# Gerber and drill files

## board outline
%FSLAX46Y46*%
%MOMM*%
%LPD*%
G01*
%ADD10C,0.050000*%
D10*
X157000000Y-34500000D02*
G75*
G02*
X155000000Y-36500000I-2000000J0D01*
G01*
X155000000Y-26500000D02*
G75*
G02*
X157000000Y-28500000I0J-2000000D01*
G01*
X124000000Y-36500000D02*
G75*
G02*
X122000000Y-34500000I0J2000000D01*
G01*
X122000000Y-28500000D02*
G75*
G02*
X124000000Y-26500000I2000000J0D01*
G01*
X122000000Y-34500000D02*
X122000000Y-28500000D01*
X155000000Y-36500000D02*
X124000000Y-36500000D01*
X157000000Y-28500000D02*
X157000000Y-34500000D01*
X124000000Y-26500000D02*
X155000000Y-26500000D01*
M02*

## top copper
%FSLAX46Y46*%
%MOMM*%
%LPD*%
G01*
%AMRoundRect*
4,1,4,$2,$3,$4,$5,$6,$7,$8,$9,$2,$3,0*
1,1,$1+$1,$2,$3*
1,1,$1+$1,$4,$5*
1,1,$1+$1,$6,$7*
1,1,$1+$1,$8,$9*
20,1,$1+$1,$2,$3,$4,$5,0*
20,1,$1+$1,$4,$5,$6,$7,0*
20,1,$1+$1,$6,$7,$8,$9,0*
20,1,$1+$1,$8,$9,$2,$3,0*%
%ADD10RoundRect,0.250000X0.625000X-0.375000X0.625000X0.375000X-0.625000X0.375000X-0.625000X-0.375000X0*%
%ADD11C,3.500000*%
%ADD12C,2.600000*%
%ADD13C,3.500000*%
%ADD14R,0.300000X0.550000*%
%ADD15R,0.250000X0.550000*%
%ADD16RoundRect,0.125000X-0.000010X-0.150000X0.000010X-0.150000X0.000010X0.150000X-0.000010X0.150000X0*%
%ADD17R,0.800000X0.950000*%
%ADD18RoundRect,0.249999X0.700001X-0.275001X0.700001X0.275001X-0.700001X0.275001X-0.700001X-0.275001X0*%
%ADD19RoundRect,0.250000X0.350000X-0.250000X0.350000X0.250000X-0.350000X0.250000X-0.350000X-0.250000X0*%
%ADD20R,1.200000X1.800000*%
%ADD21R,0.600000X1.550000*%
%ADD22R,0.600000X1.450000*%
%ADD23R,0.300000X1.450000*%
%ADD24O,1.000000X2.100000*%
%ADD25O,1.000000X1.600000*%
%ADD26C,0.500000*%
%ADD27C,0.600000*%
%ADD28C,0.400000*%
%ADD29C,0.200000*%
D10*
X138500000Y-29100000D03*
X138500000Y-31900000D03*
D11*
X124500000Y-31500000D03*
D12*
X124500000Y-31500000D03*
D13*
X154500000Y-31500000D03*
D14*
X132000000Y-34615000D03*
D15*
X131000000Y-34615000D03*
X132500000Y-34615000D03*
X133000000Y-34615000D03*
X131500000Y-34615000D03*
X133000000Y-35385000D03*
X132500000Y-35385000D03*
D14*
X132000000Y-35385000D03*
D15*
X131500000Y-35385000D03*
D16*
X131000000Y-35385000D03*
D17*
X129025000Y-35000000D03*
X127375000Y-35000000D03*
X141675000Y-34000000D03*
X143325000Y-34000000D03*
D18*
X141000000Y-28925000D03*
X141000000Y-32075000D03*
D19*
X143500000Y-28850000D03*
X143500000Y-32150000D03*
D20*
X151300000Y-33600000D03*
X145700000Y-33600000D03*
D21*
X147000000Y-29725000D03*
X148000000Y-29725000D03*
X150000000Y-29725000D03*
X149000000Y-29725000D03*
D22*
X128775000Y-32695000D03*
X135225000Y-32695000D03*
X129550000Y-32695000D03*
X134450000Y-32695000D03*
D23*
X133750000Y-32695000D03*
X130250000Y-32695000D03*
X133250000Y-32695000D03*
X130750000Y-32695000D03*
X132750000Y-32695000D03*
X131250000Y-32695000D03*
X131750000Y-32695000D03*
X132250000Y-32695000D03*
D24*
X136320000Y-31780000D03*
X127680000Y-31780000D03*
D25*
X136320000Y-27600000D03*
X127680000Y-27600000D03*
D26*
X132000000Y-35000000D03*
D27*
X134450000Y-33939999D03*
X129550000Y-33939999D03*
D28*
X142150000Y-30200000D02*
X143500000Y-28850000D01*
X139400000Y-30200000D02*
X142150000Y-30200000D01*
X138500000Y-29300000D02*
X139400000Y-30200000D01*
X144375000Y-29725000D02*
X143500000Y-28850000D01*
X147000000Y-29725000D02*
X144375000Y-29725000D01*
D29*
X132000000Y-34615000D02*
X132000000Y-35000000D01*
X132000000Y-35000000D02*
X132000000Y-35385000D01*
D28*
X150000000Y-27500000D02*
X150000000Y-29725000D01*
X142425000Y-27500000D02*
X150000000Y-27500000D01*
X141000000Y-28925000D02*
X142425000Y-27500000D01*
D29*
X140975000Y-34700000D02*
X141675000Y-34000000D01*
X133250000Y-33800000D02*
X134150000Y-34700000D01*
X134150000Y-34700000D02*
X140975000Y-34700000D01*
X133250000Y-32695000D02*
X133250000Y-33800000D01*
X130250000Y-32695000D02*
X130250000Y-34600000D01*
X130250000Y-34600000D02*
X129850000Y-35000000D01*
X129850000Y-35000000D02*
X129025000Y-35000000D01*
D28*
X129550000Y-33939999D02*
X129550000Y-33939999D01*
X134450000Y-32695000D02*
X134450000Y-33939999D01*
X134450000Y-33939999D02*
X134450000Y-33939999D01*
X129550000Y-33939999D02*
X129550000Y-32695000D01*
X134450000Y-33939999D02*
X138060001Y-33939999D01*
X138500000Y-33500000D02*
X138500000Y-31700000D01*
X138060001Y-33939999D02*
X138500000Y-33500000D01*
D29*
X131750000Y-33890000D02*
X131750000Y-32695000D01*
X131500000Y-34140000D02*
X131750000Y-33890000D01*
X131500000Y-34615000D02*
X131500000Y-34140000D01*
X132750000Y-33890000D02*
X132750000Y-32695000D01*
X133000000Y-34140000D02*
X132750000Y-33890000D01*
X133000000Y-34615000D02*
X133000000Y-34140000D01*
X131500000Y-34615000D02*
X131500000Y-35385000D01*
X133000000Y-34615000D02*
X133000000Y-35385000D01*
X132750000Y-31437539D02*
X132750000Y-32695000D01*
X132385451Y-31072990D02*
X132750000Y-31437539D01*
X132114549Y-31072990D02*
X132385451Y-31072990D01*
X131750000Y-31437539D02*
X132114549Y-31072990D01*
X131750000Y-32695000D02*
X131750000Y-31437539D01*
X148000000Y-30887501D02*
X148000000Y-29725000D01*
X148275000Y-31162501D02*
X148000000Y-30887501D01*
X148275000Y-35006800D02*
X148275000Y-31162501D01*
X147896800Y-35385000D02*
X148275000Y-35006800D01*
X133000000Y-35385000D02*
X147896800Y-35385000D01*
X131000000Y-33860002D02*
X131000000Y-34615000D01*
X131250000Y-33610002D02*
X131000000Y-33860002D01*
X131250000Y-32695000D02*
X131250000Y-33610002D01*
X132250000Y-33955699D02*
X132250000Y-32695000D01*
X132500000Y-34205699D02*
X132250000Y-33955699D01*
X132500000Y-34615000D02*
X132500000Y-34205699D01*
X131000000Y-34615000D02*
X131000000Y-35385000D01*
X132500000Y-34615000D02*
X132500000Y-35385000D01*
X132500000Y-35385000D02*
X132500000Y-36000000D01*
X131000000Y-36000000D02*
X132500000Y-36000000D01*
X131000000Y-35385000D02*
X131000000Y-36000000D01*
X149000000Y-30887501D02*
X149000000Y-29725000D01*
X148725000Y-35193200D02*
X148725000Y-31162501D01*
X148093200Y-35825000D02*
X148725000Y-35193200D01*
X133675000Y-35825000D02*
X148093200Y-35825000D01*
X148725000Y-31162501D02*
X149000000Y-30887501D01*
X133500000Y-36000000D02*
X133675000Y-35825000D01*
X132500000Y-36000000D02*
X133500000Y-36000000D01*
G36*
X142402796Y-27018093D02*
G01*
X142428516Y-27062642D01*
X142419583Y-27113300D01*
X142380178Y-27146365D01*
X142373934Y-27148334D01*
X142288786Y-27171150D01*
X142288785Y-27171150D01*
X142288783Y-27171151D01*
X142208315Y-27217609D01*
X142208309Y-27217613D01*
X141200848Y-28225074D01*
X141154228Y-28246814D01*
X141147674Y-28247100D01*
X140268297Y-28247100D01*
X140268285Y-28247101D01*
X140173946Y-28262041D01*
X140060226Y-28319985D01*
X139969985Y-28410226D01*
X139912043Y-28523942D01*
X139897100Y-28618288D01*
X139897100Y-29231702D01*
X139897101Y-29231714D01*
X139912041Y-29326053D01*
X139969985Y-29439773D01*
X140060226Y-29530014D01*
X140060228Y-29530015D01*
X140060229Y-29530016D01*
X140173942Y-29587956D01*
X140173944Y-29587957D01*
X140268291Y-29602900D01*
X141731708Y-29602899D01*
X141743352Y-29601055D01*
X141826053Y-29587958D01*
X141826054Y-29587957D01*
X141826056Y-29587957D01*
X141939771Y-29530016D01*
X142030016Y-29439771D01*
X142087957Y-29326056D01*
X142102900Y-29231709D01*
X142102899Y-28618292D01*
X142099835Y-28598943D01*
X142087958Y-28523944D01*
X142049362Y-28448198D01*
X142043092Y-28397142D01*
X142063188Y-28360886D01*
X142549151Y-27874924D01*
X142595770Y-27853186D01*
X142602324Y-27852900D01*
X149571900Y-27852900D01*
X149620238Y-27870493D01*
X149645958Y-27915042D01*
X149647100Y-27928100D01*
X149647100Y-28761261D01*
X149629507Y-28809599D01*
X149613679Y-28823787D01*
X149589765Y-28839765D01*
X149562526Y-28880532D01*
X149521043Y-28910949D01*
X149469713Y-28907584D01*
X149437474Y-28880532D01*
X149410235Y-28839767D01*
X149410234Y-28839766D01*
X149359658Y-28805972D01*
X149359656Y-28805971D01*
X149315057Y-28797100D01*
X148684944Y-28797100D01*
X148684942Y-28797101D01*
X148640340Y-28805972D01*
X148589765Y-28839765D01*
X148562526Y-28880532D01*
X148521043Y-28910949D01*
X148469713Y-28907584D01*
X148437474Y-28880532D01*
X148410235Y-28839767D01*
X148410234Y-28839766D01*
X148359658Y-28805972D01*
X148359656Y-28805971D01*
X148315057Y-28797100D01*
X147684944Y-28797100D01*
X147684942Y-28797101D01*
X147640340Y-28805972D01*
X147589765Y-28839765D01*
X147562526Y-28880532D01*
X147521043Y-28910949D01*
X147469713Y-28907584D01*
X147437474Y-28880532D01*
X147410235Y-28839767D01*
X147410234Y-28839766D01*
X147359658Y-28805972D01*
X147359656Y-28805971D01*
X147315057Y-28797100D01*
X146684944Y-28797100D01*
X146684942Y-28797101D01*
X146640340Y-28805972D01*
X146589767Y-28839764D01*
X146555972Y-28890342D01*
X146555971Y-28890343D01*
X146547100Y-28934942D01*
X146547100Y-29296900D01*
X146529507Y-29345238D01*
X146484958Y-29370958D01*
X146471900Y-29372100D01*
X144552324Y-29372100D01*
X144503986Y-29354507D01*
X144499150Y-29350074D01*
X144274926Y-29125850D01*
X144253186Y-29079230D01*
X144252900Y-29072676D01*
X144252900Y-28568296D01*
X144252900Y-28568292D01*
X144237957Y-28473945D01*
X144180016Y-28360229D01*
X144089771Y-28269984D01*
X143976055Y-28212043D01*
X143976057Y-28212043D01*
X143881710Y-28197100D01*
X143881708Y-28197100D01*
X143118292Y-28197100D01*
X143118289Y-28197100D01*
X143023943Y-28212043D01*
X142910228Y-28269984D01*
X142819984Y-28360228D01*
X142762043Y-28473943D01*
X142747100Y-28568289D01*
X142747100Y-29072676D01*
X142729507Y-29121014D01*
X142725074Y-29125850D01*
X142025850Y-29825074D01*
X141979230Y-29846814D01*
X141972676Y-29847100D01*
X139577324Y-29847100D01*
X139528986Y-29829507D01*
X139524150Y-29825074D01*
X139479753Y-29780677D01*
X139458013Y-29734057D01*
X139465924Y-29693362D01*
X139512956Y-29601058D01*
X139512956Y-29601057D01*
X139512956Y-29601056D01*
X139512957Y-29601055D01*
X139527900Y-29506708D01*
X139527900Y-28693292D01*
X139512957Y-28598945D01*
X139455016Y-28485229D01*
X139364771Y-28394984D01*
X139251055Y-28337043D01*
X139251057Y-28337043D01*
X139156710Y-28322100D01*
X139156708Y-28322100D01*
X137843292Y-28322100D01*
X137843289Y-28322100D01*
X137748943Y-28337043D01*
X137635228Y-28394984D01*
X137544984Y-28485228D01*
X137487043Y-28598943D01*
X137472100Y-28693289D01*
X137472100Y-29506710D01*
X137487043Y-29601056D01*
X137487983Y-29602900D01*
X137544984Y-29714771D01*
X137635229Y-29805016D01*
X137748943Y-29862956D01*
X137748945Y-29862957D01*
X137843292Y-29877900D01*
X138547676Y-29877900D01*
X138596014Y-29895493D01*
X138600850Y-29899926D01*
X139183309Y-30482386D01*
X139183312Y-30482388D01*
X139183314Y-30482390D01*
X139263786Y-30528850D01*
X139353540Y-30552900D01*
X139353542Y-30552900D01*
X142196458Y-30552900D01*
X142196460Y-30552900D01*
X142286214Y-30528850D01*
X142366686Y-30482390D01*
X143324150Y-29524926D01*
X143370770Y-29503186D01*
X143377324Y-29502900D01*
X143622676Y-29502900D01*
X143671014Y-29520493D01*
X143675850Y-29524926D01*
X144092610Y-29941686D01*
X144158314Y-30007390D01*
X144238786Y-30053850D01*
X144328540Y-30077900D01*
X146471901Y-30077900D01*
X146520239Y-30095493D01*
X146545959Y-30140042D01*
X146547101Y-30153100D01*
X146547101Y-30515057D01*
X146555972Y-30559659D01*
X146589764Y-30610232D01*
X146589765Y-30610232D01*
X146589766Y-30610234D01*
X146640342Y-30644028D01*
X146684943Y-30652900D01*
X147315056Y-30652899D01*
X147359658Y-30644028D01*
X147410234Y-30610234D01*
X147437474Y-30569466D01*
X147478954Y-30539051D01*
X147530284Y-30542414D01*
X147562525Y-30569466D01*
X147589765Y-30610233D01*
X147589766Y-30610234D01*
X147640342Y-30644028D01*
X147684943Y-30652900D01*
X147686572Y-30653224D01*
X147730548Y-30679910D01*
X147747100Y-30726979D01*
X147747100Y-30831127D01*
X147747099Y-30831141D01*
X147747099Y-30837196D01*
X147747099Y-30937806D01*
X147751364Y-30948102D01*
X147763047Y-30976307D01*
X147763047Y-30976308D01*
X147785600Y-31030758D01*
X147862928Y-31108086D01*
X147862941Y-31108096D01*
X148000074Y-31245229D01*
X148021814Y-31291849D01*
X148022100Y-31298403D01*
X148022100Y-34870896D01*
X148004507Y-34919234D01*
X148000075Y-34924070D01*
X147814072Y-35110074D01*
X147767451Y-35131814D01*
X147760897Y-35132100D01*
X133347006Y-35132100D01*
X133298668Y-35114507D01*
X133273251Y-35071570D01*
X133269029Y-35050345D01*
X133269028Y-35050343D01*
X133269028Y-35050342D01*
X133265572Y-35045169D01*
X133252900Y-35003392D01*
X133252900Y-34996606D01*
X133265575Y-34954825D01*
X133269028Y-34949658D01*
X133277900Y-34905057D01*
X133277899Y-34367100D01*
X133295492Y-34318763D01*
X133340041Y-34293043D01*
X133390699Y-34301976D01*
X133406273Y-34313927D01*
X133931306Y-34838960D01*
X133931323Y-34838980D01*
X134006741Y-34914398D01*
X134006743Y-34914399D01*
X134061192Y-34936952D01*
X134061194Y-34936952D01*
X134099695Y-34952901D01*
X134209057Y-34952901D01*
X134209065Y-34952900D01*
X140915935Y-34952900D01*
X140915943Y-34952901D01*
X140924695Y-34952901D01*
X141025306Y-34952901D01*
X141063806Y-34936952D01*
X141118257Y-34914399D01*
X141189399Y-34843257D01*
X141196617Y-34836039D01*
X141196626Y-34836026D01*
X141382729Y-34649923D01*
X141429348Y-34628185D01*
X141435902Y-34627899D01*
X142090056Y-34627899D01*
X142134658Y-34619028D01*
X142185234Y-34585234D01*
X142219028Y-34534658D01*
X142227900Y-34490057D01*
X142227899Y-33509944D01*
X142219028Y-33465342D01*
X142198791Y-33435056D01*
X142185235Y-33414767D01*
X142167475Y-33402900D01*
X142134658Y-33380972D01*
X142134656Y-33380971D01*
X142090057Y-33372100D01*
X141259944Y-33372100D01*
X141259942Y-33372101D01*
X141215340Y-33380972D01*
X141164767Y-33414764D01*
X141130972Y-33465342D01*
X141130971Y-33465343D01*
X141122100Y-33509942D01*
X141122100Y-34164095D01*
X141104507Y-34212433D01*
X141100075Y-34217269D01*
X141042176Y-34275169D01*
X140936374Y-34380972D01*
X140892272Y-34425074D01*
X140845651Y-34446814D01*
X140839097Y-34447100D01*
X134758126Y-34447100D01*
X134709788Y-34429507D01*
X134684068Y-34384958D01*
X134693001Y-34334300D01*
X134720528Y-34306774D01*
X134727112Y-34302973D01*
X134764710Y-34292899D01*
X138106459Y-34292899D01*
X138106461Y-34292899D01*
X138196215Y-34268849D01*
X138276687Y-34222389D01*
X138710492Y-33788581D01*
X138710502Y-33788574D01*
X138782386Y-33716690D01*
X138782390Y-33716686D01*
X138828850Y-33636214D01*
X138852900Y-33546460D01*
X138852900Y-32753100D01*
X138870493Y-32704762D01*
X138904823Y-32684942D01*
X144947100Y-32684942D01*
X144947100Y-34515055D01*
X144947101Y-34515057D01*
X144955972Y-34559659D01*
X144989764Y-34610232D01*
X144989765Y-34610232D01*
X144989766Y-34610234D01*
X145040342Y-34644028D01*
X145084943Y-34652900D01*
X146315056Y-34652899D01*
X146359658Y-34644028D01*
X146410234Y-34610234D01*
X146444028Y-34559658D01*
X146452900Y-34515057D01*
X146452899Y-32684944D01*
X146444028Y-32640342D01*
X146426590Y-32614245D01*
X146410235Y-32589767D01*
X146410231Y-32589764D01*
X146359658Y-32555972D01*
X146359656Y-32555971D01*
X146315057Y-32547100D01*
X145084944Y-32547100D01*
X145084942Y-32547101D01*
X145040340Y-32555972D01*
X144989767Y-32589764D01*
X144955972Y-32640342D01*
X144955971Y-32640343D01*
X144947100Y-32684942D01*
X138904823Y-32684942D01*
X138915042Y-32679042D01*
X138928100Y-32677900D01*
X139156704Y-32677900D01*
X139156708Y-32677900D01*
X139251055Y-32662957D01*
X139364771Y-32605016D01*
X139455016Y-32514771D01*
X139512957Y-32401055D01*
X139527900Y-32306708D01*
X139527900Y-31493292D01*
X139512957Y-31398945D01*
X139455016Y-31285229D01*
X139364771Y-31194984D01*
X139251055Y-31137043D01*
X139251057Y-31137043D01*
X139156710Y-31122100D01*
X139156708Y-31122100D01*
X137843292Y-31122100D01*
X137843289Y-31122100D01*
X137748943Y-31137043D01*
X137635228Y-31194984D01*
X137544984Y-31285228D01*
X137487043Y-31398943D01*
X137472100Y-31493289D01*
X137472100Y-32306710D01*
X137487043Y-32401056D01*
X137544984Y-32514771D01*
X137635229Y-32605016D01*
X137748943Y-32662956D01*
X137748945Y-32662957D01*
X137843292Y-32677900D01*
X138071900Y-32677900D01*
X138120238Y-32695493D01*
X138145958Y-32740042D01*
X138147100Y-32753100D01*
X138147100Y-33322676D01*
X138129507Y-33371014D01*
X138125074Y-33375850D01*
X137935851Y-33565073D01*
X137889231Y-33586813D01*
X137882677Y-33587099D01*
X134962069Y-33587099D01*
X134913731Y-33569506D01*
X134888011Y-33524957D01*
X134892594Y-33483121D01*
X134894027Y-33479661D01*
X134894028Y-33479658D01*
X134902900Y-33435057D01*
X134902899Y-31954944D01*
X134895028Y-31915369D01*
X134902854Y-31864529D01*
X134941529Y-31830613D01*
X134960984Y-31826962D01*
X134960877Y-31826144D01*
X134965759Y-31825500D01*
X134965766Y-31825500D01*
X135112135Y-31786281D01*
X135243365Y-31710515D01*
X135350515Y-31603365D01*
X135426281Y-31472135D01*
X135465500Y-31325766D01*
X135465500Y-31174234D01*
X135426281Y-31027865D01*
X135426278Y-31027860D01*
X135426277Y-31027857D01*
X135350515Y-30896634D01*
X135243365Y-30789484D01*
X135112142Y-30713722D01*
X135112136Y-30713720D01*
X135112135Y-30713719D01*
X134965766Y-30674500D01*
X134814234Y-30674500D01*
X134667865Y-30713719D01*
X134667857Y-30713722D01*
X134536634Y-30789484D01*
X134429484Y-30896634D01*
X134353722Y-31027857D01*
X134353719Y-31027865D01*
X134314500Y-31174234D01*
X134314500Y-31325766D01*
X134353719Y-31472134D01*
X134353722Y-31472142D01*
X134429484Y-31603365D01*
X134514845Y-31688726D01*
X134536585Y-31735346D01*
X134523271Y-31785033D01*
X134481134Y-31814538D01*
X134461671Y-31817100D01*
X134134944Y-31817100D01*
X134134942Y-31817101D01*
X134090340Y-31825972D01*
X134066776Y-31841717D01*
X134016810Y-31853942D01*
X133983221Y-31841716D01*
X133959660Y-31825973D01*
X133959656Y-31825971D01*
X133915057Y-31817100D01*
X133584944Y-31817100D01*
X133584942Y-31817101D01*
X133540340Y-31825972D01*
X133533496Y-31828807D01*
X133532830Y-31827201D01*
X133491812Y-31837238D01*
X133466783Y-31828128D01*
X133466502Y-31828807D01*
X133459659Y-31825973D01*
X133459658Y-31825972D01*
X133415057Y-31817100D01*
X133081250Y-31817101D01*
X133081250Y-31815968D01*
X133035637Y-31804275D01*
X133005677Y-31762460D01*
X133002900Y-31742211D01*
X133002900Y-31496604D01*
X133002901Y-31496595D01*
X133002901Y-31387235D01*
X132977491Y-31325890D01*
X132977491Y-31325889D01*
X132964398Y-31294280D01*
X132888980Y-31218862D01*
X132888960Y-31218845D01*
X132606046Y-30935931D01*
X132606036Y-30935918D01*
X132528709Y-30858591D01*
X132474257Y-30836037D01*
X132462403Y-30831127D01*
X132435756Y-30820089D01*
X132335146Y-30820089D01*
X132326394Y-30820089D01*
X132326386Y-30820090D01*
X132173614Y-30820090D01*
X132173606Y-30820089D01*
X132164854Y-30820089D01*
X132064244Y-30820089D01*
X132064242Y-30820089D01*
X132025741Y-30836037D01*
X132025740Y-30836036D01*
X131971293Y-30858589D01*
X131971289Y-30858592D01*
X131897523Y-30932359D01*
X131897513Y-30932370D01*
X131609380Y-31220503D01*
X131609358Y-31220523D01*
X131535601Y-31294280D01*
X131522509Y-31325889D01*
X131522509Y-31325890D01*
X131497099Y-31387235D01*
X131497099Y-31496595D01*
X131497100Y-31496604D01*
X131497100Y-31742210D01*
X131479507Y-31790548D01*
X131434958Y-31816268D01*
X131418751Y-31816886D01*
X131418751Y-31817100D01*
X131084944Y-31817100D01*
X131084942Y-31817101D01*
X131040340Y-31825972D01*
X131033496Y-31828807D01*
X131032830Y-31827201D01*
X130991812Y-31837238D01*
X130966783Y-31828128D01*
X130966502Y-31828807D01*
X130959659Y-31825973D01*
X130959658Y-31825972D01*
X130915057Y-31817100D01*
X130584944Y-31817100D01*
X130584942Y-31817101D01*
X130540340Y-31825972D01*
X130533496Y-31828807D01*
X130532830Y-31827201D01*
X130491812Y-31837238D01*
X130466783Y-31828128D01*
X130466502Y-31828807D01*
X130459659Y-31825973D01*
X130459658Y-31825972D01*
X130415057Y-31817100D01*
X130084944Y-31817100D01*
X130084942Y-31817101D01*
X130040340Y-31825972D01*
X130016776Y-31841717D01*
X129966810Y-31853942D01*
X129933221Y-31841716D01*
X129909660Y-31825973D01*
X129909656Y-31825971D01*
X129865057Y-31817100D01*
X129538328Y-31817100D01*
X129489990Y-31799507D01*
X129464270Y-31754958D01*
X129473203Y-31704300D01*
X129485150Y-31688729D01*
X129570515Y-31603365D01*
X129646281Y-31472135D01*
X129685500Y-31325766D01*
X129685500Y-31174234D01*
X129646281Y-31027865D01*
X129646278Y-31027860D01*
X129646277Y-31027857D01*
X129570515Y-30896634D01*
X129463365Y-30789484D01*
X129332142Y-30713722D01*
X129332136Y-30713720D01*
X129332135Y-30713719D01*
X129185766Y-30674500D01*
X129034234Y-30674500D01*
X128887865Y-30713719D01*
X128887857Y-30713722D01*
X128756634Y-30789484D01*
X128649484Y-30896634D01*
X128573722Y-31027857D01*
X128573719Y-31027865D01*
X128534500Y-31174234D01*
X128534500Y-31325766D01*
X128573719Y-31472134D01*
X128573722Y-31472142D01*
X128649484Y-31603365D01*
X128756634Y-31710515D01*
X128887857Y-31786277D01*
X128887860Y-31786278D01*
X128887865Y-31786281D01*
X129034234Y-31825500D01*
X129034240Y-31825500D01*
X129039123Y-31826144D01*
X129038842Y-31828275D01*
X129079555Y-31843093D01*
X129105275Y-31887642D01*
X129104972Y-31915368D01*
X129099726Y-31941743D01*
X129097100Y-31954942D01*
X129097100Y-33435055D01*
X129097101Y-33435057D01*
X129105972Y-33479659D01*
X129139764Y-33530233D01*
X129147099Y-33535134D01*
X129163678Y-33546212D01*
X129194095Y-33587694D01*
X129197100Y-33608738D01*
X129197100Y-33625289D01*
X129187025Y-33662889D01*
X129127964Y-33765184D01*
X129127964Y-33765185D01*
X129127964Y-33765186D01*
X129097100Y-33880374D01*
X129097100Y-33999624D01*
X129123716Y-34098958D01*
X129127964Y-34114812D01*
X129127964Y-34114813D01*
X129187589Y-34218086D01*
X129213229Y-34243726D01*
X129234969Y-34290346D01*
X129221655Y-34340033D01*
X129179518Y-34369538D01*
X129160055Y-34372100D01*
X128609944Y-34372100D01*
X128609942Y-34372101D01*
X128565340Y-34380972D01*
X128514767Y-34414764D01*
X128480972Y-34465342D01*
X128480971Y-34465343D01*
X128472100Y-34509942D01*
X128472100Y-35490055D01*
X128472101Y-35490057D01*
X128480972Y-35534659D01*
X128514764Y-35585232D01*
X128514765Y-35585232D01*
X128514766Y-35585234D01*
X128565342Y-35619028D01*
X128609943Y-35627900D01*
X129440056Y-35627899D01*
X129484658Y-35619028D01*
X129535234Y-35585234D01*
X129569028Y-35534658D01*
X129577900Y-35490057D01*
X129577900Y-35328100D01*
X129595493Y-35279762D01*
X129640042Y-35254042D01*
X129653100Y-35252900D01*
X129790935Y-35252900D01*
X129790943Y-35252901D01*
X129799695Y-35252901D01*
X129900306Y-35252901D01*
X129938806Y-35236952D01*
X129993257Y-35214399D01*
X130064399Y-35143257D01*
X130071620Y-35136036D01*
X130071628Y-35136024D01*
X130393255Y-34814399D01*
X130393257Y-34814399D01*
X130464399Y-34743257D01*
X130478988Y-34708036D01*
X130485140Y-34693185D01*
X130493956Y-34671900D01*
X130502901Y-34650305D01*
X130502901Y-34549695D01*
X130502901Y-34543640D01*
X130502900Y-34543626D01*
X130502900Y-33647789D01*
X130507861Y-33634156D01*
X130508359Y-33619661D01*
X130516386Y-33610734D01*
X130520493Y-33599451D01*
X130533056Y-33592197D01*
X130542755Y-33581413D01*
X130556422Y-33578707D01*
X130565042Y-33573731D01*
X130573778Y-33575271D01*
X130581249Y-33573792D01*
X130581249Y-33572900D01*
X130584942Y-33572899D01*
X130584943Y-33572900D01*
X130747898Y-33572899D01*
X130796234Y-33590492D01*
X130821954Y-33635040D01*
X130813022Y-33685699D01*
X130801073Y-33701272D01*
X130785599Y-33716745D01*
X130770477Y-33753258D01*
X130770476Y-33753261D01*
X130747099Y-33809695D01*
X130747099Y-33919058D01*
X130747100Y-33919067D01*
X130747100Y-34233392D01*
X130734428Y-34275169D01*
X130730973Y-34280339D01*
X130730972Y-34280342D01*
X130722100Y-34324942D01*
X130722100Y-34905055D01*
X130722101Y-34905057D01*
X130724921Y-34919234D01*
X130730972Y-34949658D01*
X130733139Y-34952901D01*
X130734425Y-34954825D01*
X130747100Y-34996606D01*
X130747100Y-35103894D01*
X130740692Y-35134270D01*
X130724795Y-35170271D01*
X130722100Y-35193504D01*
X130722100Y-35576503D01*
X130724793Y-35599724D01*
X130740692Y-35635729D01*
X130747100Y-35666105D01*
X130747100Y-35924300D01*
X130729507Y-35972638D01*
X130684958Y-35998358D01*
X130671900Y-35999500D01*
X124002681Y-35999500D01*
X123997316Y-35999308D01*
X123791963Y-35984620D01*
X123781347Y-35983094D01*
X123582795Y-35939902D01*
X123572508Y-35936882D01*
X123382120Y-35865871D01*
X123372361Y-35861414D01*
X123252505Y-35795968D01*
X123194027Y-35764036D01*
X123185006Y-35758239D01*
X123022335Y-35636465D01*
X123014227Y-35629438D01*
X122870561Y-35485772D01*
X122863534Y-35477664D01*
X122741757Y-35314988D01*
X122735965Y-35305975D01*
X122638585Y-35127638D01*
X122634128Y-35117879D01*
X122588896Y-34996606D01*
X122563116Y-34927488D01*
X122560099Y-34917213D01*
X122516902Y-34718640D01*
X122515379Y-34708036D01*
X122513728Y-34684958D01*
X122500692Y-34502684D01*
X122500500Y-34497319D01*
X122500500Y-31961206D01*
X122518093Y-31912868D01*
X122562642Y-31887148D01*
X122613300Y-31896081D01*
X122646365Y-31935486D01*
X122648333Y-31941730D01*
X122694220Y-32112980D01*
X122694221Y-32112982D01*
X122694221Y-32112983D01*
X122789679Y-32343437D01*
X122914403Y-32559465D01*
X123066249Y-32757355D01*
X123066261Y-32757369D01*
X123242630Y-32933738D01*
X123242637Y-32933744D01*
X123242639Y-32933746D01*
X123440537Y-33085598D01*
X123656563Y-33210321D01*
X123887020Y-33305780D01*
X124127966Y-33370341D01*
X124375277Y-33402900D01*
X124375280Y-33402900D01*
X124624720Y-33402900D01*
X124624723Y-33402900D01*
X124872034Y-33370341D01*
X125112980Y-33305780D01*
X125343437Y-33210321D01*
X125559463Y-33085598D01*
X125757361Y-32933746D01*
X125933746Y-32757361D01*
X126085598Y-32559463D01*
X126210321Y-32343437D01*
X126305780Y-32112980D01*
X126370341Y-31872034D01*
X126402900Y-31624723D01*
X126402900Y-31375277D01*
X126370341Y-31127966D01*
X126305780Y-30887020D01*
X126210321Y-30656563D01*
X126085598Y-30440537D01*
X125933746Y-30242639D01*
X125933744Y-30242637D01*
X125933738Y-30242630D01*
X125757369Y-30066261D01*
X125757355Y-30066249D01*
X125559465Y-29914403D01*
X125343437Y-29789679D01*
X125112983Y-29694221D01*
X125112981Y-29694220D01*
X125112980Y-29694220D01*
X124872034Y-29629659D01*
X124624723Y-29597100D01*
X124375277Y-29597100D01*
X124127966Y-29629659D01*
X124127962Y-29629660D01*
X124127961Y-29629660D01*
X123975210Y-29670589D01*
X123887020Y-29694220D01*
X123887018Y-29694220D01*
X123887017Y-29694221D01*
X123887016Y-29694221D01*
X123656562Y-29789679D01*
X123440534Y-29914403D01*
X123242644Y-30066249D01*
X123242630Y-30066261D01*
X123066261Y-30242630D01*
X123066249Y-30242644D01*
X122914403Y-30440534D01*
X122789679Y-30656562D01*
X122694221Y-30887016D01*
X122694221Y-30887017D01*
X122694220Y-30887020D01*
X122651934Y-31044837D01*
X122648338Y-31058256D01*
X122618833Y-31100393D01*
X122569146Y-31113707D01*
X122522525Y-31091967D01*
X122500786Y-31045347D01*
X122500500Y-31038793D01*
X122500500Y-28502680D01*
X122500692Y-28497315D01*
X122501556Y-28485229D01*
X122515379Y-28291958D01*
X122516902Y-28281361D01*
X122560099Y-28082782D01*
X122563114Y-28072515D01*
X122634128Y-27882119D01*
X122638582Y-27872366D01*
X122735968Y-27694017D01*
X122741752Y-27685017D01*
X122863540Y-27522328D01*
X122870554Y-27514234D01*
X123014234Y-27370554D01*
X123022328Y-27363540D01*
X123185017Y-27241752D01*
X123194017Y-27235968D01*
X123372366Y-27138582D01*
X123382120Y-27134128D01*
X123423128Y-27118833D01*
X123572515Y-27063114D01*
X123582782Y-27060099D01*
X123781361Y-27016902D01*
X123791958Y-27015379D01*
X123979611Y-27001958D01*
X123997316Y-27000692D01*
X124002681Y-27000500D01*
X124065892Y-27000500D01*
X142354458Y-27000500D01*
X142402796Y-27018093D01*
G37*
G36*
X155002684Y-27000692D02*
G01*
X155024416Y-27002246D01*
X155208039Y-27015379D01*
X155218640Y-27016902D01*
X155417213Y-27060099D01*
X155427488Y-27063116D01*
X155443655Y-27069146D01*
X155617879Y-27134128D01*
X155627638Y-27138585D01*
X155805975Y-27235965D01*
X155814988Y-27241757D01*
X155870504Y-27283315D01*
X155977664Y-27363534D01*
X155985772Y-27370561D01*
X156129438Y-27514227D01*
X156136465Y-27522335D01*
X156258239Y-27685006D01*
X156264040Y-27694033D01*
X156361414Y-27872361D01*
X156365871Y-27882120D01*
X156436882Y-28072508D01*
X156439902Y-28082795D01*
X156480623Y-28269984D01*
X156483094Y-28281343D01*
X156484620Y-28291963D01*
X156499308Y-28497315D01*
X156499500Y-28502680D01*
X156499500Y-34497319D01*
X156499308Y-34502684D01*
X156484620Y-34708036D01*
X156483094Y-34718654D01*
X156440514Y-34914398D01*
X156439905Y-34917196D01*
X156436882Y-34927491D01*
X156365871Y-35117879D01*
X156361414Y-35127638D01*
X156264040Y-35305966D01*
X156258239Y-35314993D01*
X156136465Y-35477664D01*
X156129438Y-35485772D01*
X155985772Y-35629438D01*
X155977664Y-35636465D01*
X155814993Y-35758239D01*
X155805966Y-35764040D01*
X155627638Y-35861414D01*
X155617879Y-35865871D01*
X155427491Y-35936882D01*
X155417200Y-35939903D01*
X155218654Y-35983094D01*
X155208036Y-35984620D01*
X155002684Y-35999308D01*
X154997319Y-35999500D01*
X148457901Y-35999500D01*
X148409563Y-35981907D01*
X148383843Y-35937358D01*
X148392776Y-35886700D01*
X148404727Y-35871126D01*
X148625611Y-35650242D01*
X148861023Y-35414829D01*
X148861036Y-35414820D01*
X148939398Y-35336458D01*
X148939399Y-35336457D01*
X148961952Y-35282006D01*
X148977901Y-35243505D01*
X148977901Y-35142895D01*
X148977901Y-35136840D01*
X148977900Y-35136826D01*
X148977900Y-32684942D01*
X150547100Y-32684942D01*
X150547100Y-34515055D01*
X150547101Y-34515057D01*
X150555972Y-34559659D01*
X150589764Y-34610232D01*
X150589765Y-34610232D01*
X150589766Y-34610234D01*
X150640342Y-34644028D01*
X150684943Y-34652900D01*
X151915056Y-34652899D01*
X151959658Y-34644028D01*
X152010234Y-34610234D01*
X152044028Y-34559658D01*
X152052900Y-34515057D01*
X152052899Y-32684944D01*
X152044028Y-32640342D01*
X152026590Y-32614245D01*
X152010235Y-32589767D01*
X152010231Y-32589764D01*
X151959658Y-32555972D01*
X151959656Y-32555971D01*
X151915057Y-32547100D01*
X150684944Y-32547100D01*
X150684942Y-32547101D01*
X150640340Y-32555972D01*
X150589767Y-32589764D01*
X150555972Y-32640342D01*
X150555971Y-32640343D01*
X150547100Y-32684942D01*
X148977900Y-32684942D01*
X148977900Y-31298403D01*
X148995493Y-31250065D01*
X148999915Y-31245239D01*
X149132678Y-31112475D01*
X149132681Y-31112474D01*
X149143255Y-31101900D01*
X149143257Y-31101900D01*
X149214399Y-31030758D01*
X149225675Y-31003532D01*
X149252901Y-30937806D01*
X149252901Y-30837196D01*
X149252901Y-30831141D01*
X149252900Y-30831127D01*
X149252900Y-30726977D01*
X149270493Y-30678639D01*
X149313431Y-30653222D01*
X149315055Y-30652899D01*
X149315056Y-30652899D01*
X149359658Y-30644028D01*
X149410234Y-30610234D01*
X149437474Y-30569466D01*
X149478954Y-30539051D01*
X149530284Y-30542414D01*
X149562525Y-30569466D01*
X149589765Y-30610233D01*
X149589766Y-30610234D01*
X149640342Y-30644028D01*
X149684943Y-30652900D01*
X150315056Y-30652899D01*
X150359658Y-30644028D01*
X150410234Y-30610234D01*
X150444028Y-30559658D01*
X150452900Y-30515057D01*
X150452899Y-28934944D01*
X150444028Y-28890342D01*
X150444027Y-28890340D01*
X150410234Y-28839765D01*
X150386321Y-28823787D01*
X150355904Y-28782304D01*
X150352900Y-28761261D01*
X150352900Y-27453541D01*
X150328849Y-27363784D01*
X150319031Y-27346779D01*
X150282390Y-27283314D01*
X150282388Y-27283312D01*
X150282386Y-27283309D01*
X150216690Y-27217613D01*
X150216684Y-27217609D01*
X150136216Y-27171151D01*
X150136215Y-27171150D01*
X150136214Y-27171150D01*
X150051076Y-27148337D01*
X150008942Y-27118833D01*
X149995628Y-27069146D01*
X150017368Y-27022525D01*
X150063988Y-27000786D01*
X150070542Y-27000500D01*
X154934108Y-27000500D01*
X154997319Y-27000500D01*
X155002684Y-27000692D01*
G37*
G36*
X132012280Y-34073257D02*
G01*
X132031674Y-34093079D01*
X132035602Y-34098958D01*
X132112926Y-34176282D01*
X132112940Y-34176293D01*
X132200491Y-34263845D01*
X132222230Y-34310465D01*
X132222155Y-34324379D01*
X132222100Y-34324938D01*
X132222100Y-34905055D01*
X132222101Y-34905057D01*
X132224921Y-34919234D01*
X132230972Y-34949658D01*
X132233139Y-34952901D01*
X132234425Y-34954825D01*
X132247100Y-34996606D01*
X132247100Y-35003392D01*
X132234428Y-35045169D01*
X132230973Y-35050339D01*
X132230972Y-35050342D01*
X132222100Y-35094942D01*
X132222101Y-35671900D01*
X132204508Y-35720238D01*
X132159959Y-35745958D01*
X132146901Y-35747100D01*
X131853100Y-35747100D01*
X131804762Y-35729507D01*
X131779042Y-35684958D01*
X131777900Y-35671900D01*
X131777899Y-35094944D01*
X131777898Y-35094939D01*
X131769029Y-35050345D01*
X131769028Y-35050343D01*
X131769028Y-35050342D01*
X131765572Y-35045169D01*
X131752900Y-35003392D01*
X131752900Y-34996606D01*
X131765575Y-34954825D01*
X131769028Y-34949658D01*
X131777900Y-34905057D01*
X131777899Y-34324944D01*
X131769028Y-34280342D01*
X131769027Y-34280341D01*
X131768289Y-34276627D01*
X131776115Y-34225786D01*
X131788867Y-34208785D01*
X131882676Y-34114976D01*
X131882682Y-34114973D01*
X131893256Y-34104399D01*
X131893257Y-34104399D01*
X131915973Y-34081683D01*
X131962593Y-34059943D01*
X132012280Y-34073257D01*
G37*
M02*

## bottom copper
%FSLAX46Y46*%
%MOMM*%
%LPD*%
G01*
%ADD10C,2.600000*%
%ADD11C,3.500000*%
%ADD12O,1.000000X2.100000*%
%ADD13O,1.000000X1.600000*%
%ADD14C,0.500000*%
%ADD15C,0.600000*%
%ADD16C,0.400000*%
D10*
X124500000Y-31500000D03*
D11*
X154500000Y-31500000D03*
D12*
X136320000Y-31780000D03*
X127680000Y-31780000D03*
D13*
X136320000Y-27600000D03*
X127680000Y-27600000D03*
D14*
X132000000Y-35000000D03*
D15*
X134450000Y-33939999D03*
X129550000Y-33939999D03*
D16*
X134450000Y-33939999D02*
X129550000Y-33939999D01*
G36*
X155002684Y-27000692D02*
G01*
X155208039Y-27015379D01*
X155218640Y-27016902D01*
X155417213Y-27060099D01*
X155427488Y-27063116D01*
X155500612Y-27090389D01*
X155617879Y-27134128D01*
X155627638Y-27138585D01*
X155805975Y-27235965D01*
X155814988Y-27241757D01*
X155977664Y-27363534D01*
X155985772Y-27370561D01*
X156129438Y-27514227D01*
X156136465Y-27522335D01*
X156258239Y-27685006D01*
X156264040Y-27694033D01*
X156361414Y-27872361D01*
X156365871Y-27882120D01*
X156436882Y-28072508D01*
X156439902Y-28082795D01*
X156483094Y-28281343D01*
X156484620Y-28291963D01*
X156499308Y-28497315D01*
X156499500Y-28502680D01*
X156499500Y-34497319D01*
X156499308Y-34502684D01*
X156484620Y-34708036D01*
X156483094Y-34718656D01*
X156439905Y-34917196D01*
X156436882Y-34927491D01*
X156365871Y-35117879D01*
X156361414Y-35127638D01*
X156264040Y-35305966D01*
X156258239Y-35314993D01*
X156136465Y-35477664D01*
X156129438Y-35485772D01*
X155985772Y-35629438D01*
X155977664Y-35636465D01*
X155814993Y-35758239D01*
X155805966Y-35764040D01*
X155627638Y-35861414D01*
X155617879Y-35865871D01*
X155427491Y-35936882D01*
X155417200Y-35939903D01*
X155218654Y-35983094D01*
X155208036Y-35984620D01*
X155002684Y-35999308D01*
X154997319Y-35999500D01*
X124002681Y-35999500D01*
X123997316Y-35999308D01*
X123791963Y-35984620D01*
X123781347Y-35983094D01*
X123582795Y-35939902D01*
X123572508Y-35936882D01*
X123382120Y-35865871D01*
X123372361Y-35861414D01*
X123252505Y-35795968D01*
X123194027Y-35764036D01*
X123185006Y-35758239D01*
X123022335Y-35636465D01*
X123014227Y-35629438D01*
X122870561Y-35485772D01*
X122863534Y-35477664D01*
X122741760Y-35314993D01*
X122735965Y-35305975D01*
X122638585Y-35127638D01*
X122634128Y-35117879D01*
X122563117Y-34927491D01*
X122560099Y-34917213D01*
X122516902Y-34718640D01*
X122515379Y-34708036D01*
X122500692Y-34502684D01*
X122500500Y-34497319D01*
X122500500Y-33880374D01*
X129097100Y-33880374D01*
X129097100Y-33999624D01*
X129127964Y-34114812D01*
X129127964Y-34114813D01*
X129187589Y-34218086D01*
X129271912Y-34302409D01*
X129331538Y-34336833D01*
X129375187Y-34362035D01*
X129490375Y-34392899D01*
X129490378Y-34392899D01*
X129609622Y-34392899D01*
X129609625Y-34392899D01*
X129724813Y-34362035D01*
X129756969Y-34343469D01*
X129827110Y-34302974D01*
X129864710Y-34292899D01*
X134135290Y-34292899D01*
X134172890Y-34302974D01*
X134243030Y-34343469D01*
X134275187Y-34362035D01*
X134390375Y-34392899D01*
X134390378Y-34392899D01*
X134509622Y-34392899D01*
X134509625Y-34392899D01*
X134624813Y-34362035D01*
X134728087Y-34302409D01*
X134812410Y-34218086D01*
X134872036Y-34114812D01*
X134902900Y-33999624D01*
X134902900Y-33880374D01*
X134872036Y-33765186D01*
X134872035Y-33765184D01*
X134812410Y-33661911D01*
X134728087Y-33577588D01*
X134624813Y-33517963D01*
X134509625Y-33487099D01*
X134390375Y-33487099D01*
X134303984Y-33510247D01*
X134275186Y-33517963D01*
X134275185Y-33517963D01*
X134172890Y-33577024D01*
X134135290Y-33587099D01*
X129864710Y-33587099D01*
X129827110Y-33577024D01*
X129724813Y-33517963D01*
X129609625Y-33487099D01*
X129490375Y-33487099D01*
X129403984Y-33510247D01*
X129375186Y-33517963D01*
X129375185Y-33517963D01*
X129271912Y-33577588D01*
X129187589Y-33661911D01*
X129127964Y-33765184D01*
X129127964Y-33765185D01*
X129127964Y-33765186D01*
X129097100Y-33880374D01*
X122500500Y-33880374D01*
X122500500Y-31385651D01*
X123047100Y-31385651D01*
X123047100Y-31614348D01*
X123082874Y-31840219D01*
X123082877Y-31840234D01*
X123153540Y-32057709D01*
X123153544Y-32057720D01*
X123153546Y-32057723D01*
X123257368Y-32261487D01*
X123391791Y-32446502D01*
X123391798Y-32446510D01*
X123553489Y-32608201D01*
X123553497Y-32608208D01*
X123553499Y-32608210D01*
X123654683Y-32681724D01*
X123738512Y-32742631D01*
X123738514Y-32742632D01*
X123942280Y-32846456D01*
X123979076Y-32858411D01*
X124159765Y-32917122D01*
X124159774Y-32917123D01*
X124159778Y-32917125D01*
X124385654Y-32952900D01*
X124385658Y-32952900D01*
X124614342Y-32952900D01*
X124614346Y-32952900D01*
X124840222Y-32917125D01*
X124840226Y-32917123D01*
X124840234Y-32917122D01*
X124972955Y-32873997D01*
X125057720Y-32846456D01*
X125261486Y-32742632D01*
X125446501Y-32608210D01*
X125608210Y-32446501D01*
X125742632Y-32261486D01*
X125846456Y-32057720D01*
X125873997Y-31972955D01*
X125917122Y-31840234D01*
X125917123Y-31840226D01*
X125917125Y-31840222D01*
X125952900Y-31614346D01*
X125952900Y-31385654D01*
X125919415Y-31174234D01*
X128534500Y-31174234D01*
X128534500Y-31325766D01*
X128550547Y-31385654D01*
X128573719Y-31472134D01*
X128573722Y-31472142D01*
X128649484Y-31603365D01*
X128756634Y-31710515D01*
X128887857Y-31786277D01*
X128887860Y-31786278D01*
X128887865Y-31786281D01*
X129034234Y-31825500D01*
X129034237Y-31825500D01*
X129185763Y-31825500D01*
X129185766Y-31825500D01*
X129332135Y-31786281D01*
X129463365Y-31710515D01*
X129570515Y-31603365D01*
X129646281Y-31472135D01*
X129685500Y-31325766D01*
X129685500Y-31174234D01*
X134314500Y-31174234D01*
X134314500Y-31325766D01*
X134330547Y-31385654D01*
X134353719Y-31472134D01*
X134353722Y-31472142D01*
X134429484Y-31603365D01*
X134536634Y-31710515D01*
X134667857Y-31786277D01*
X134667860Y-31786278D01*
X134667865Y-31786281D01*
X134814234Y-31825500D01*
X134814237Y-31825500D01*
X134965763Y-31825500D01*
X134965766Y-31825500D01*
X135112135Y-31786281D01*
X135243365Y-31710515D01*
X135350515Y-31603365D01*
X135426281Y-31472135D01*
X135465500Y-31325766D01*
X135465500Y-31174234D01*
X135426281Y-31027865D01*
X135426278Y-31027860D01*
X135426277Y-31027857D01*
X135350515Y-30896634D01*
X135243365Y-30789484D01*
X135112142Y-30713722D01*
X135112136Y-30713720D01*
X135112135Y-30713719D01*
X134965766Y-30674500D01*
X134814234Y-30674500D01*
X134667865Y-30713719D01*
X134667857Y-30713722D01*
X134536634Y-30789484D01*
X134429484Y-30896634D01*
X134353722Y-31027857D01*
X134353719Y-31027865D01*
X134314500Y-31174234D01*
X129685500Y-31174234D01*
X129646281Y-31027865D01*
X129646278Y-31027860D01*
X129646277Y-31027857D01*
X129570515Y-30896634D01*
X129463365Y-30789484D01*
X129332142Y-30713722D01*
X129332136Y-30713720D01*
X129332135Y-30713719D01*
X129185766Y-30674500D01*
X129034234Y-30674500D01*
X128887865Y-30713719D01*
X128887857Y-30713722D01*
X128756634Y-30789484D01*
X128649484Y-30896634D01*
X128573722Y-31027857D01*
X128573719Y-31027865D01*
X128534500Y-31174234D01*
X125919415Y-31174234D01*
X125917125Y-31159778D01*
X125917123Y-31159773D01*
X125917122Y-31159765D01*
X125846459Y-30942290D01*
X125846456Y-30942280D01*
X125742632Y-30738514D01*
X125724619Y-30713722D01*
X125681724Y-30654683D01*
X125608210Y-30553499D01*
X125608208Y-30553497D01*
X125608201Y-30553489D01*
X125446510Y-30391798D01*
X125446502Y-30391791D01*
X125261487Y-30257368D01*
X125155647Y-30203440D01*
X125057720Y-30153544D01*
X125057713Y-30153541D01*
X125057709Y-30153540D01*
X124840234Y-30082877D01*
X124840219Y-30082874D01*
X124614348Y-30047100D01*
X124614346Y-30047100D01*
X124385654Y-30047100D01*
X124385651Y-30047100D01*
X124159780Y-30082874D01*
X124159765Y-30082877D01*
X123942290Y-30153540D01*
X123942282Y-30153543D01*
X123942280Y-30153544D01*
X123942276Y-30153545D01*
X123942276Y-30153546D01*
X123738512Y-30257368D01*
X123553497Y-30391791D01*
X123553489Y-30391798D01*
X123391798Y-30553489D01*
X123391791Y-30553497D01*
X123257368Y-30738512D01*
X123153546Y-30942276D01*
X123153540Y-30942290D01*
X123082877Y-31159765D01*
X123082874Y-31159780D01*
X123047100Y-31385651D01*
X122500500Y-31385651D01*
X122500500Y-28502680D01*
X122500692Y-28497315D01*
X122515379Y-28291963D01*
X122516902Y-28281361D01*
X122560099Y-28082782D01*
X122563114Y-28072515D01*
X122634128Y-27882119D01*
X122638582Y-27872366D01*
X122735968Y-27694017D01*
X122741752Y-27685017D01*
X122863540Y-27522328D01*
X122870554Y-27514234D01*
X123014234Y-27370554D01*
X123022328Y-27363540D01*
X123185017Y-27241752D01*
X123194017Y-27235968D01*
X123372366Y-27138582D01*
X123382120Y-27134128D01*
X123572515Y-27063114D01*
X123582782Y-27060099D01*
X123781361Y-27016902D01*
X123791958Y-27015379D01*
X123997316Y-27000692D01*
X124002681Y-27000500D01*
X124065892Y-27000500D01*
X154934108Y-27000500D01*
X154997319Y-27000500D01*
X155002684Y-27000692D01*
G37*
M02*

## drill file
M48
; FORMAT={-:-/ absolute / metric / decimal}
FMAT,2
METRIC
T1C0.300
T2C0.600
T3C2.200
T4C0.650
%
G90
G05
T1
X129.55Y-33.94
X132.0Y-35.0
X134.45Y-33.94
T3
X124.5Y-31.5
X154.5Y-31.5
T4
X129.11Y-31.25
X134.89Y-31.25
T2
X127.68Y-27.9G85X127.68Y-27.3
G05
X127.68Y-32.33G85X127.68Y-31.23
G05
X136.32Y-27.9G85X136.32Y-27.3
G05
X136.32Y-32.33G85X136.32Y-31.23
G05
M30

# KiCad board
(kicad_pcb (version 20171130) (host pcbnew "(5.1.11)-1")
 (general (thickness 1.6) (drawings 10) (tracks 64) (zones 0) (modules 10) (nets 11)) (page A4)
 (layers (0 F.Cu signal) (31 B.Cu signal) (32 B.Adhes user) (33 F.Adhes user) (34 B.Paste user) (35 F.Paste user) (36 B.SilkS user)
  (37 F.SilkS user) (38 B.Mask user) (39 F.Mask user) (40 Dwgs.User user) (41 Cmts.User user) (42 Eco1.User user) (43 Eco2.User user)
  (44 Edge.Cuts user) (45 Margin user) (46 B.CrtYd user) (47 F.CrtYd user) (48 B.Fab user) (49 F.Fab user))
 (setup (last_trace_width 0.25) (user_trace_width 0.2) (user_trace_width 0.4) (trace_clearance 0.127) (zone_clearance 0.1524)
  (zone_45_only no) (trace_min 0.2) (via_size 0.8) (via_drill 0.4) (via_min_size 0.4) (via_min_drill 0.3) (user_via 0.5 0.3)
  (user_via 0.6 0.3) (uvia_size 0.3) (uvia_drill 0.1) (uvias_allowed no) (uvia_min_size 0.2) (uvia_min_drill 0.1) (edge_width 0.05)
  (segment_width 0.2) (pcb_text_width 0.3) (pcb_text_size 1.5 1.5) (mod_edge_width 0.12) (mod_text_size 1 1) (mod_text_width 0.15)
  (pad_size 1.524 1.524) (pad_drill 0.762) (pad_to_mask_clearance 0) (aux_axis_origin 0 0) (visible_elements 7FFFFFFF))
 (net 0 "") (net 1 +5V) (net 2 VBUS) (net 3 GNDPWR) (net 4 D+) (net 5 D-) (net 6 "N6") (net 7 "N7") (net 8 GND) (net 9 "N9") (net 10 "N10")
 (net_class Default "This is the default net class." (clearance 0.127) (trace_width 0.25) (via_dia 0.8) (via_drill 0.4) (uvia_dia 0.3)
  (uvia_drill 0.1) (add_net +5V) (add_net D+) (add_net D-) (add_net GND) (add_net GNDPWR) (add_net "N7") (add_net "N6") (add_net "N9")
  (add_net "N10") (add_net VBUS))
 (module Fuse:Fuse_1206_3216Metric (layer F.Cu) (at 138.5 30.5 90)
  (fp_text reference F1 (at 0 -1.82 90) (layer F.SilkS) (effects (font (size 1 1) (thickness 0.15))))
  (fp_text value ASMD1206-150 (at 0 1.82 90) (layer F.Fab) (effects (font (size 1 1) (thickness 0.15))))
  (pad 2 smd roundrect (at 1.4 0 90) (size 1.25 1.75) (layers F.Cu F.Paste F.Mask) (roundrect_rratio 0.2) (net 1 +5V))
  (pad 1 smd roundrect (at -1.4 0 90) (size 1.25 1.75) (layers F.Cu F.Paste F.Mask) (roundrect_rratio 0.2) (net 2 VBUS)))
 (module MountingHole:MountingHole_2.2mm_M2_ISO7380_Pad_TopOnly (layer F.Cu) (at 124.5 31.5)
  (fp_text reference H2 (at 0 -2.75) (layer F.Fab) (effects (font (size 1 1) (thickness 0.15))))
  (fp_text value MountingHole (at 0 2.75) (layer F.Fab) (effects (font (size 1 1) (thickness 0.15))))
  (pad 1 connect circle (at 0 0) (size 3.5 3.5) (layers F.Cu F.Mask))
  (pad 1 thru_hole circle (at 0 0) (size 2.6 2.6) (drill 2.2) (layers *.Cu *.Mask)))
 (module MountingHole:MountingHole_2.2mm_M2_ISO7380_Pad (layer F.Cu) (at 154.5 31.5)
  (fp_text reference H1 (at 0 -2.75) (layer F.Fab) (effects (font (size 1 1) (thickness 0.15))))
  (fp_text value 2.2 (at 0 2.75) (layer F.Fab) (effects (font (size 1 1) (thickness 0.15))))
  (pad 1 thru_hole circle (at 0 0) (size 3.5 3.5) (drill 2.2) (layers *.Cu *.Mask) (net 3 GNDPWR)))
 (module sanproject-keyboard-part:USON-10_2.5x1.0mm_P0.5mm (layer F.Cu) (at 132 35 90)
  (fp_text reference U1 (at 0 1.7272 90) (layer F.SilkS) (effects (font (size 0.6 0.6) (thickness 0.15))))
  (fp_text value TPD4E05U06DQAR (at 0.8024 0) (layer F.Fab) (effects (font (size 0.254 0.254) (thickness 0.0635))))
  (pad 8 smd rect (at 0.385 0) (size 0.3 0.55) (layers F.Cu F.Paste F.Mask) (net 3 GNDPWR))
  (pad 10 smd rect (at 0.385 -1) (size 0.25 0.55) (layers F.Cu F.Paste F.Mask) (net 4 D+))
  (pad 7 smd rect (at 0.385 0.5) (size 0.25 0.55) (layers F.Cu F.Paste F.Mask) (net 4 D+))
  (pad 6 smd rect (at 0.385 1) (size 0.25 0.55) (layers F.Cu F.Paste F.Mask) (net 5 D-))
  (pad 9 smd rect (at 0.385 -0.5) (size 0.25 0.55) (layers F.Cu F.Paste F.Mask) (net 5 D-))
  (pad 5 smd rect (at -0.385 1) (size 0.25 0.55) (layers F.Cu F.Paste F.Mask) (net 5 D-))
  (pad 4 smd rect (at -0.385 0.5) (size 0.25 0.55) (layers F.Cu F.Paste F.Mask) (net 4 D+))
  (pad 3 smd rect (at -0.385 0) (size 0.3 0.55) (layers F.Cu F.Paste F.Mask) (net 3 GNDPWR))
  (pad 2 smd rect (at -0.385 -0.5) (size 0.25 0.55) (layers F.Cu F.Paste F.Mask) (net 5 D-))
  (pad 1 smd roundrect (at -0.385 -1) (size 0.25 0.55) (layers F.Cu F.Paste F.Mask) (roundrect_rratio 0.5) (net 4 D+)))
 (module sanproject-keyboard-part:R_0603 (layer F.Cu) (at 128.2 35)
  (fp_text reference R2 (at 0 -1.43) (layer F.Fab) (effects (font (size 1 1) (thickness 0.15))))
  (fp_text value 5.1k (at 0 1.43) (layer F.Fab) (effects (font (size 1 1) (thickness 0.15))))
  (pad 2 smd rect (at 0.825 0) (size 0.8 0.95) (layers F.Cu F.Paste F.Mask) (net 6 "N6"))
  (pad 1 smd rect (at -0.825 0) (size 0.8 0.95) (layers F.Cu F.Paste F.Mask) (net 3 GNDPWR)))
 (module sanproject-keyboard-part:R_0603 (layer F.Cu) (at 142.5 34 180)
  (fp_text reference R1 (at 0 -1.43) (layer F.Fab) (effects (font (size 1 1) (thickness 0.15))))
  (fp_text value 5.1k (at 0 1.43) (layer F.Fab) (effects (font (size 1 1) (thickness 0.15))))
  (pad 2 smd rect (at 0.825 0 180) (size 0.8 0.95) (layers F.Cu F.Paste F.Mask) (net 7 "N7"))
  (pad 1 smd rect (at -0.825 0 180) (size 0.8 0.95) (layers F.Cu F.Paste F.Mask) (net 3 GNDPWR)))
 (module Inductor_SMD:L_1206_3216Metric (layer F.Cu) (at 141 30.5 90)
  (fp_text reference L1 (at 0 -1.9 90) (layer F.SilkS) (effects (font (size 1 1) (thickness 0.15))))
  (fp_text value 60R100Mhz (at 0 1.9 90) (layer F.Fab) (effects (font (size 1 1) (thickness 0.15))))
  (pad 2 smd roundrect (at 1.575 0 90) (size 1.05 1.9) (layers F.Cu F.Paste F.Mask) (roundrect_rratio 0.2380942857142857) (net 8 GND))
  (pad 1 smd roundrect (at -1.575 0 90) (size 1.05 1.9) (layers F.Cu F.Paste F.Mask) (roundrect_rratio 0.2380942857142857) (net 3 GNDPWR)))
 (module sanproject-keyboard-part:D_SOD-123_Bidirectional (layer F.Cu) (at 143.5 30.5 90)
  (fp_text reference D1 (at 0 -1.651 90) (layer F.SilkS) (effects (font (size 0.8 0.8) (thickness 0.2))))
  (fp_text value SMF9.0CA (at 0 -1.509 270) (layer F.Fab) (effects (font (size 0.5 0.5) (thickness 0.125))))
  (pad 2 smd roundrect (at 1.65 0 90) (size 1 1.2) (layers F.Cu F.Paste F.Mask) (roundrect_rratio 0.25) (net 1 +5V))
  (pad 1 smd roundrect (at -1.65 0 90) (size 1 1.2) (layers F.Cu F.Paste F.Mask) (roundrect_rratio 0.25) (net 3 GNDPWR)))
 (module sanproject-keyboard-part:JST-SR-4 (layer F.Cu) (at 148.5 34.5)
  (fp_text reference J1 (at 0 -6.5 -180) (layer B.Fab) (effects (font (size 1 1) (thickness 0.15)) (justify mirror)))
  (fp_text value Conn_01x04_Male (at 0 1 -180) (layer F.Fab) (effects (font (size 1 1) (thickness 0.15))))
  (pad "" smd rect (at 2.8 -0.9) (size 1.2 1.8) (layers F.Cu F.Paste F.Mask))
  (pad "" smd rect (at -2.8 -0.9) (size 1.2 1.8) (layers F.Cu F.Paste F.Mask))
  (pad 1 smd rect (at -1.5 -4.775) (size 0.6 1.55) (layers F.Cu F.Paste F.Mask) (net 1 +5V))
  (pad 2 smd rect (at -0.5 -4.775) (size 0.6 1.55) (layers F.Cu F.Paste F.Mask) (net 5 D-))
  (pad 4 smd rect (at 1.5 -4.775) (size 0.6 1.55) (layers F.Cu F.Paste F.Mask) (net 8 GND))
  (pad 3 smd rect (at 0.5 -4.775) (size 0.6 1.55) (layers F.Cu F.Paste F.Mask) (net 4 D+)))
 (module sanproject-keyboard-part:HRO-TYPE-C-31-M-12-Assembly (layer F.Cu) (at 132 25 180)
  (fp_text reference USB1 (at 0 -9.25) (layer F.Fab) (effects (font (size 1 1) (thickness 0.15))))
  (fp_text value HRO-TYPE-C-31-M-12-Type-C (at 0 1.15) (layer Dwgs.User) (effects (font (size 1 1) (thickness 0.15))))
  (pad 12 smd rect (at 3.225 -7.695 180) (size 0.6 1.45) (layers F.Cu F.Paste F.Mask) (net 3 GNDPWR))
  (pad 1 smd rect (at -3.225 -7.695 180) (size 0.6 1.45) (layers F.Cu F.Paste F.Mask) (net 3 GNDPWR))
  (pad 11 smd rect (at 2.45 -7.695 180) (size 0.6 1.45) (layers F.Cu F.Paste F.Mask) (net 2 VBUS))
  (pad 2 smd rect (at -2.45 -7.695 180) (size 0.6 1.45) (layers F.Cu F.Paste F.Mask) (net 2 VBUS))
  (pad 3 smd rect (at -1.75 -7.695 180) (size 0.3 1.45) (layers F.Cu F.Paste F.Mask) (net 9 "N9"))
  (pad 10 smd rect (at 1.75 -7.695 180) (size 0.3 1.45) (layers F.Cu F.Paste F.Mask) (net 6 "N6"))
  (pad 4 smd rect (at -1.25 -7.695 180) (size 0.3 1.45) (layers F.Cu F.Paste F.Mask) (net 7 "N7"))
  (pad 9 smd rect (at 1.25 -7.695 180) (size 0.3 1.45) (layers F.Cu F.Paste F.Mask) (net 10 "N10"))
  (pad 5 smd rect (at -0.75 -7.695 180) (size 0.3 1.45) (layers F.Cu F.Paste F.Mask) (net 5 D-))
  (pad 8 smd rect (at 0.75 -7.695 180) (size 0.3 1.45) (layers F.Cu F.Paste F.Mask) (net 4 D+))
  (pad 7 smd rect (at 0.25 -7.695 180) (size 0.3 1.45) (layers F.Cu F.Paste F.Mask) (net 5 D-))
  (pad 6 smd rect (at -0.25 -7.695 180) (size 0.3 1.45) (layers F.Cu F.Paste F.Mask) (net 4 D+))
  (pad "" np_thru_hole circle (at 2.89 -6.25 180) (size 0.65 0.65) (drill 0.65) (layers *.Cu *.Mask))
  (pad "" np_thru_hole circle (at -2.89 -6.25 180) (size 0.65 0.65) (drill 0.65) (layers *.Cu *.Mask))
  (pad 13 thru_hole oval (at -4.32 -6.78 180) (size 1 2.1) (drill oval 0.6 1.7) (layers *.Cu *.Mask) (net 3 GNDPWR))
  (pad 13 thru_hole oval (at 4.32 -6.78 180) (size 1 2.1) (drill oval 0.6 1.7) (layers *.Cu *.Mask) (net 3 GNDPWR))
  (pad 13 thru_hole oval (at -4.32 -2.6 180) (size 1 1.6) (drill oval 0.6 1.2) (layers *.Cu *.Mask) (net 3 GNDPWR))
  (pad 13 thru_hole oval (at 4.32 -2.6 180) (size 1 1.6) (drill oval 0.6 1.2) (layers *.Cu *.Mask) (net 3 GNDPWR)))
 (gr_arc (start 155 34.5) (end 155 36.5) (angle -90) (layer Edge.Cuts) (width 0.05))
 (gr_arc (start 155 28.5) (end 157 28.5) (angle -90) (layer Edge.Cuts) (width 0.05))
 (gr_arc (start 124 34.5) (end 122 34.5) (angle -90) (layer Edge.Cuts) (width 0.05))
 (gr_arc (start 124 28.5) (end 124 26.5) (angle -90) (layer Edge.Cuts) (width 0.05))
 (gr_line (start 122 34.5) (end 122 28.5) (layer Edge.Cuts) (width 0.05))
 (gr_line (start 155 36.5) (end 124 36.5) (layer Edge.Cuts) (width 0.05))
 (gr_line (start 157 28.5) (end 157 34.5) (layer Edge.Cuts) (width 0.05))
 (gr_line (start 124 26.5) (end 155 26.5) (layer Edge.Cuts) (width 0.05))
 (segment (start 142.15 30.2) (end 143.5 28.85) (width 0.4) (layer F.Cu) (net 1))
 (segment (start 139.4 30.2) (end 142.15 30.2) (width 0.4) (layer F.Cu) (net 1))
 (segment (start 138.5 29.3) (end 139.4 30.2) (width 0.4) (layer F.Cu) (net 1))
 (segment (start 144.375 29.725) (end 143.5 28.85) (width 0.4) (layer F.Cu) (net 1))
 (segment (start 147 29.725) (end 144.375 29.725) (width 0.4) (layer F.Cu) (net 1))
 (via (at 132 35) (size 0.5) (drill 0.3) (layers F.Cu B.Cu) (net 3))
 (segment (start 132 34.615) (end 132 35) (width 0.2) (layer F.Cu) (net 3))
 (segment (start 132 35) (end 132 35.385) (width 0.2) (layer F.Cu) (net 3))
 (segment (start 150 27.5) (end 150 29.725) (width 0.4) (layer F.Cu) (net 8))
 (segment (start 142.425 27.5) (end 150 27.5) (width 0.4) (layer F.Cu) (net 8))
 (segment (start 141 28.925) (end 142.425 27.5) (width 0.4) (layer F.Cu) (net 8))
 (segment (start 140.975 34.7) (end 141.675 34) (width 0.2) (layer F.Cu) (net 7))
 (segment (start 133.25 33.8) (end 134.15 34.7) (width 0.2) (layer F.Cu) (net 7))
 (segment (start 134.15 34.7) (end 140.975 34.7) (width 0.2) (layer F.Cu) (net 7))
 (segment (start 133.25 32.695) (end 133.25 33.8) (width 0.2) (layer F.Cu) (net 7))
 (segment (start 130.25 32.695) (end 130.25 34.6) (width 0.2) (layer F.Cu) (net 6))
 (segment (start 130.25 34.6) (end 129.85 35) (width 0.2) (layer F.Cu) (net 6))
 (segment (start 129.85 35) (end 129.025 35) (width 0.2) (layer F.Cu) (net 6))
 (segment (start 129.55 33.939999) (end 129.55 33.939999) (width 0.4) (layer F.Cu) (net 2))
 (segment (start 134.45 32.695) (end 134.45 33.939999) (width 0.4) (layer F.Cu) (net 2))
 (segment (start 134.45 33.939999) (end 134.45 33.939999) (width 0.4) (layer F.Cu) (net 2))
 (via (at 134.45 33.939999) (size 0.6) (drill 0.3) (layers F.Cu B.Cu) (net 2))
 (segment (start 129.55 33.939999) (end 129.55 32.695) (width 0.4) (layer F.Cu) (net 2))
 (via (at 129.55 33.939999) (size 0.6) (drill 0.3) (layers F.Cu B.Cu) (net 2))
 (segment (start 134.45 33.939999) (end 129.55 33.939999) (width 0.4) (layer B.Cu) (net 2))
 (segment (start 134.45 33.939999) (end 138.060001 33.939999) (width 0.4) (layer F.Cu) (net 2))
 (segment (start 138.5 33.5) (end 138.5 31.7) (width 0.4) (layer F.Cu) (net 2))
 (segment (start 138.060001 33.939999) (end 138.5 33.5) (width 0.4) (layer F.Cu) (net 2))
 (segment (start 131.75 33.89) (end 131.75 32.695) (width 0.2) (layer F.Cu) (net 5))
 (segment (start 131.5 34.14) (end 131.75 33.89) (width 0.2) (layer F.Cu) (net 5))
 (segment (start 131.5 34.615) (end 131.5 34.14) (width 0.2) (layer F.Cu) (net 5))
 (segment (start 132.75 33.89) (end 132.75 32.695) (width 0.2) (layer F.Cu) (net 5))
 (segment (start 133 34.14) (end 132.75 33.89) (width 0.2) (layer F.Cu) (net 5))
 (segment (start 133 34.615) (end 133 34.14) (width 0.2) (layer F.Cu) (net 5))
 (segment (start 131.5 34.615) (end 131.5 35.385) (width 0.2) (layer F.Cu) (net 5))
 (segment (start 133 34.615) (end 133 35.385) (width 0.2) (layer F.Cu) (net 5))
 (segment (start 132.75 31.437539) (end 132.75 32.695) (width 0.2) (layer F.Cu) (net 5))
 (segment (start 132.385451 31.07299) (end 132.75 31.437539) (width 0.2) (layer F.Cu) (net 5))
 (segment (start 132.114549 31.07299) (end 132.385451 31.07299) (width 0.2) (layer F.Cu) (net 5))
 (segment (start 131.75 31.437539) (end 132.114549 31.07299) (width 0.2) (layer F.Cu) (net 5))
 (segment (start 131.75 32.695) (end 131.75 31.437539) (width 0.2) (layer F.Cu) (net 5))
 (segment (start 148 30.887501) (end 148 29.725) (width 0.2) (layer F.Cu) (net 5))
 (segment (start 148.275 31.162501) (end 148 30.887501) (width 0.2) (layer F.Cu) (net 5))
 (segment (start 148.275 35.0068) (end 148.275 31.162501) (width 0.2) (layer F.Cu) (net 5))
 (segment (start 147.8968 35.385) (end 148.275 35.0068) (width 0.2) (layer F.Cu) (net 5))
 (segment (start 133 35.385) (end 147.8968 35.385) (width 0.2) (layer F.Cu) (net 5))
 (segment (start 131 33.860002) (end 131 34.615) (width 0.2) (layer F.Cu) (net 4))
 (segment (start 131.25 33.610002) (end 131 33.860002) (width 0.2) (layer F.Cu) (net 4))
 (segment (start 131.25 32.695) (end 131.25 33.610002) (width 0.2) (layer F.Cu) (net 4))
 (segment (start 132.25 33.955699) (end 132.25 32.695) (width 0.2) (layer F.Cu) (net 4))
 (segment (start 132.5 34.205699) (end 132.25 33.955699) (width 0.2) (layer F.Cu) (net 4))
 (segment (start 132.5 34.615) (end 132.5 34.205699) (width 0.2) (layer F.Cu) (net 4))
 (segment (start 131 34.615) (end 131 35.385) (width 0.2) (layer F.Cu) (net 4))
 (segment (start 132.5 34.615) (end 132.5 35.385) (width 0.2) (layer F.Cu) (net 4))
 (segment (start 132.5 35.385) (end 132.5 36) (width 0.2) (layer F.Cu) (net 4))
 (segment (start 131 36) (end 132.5 36) (width 0.2) (layer F.Cu) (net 4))
 (segment (start 131 35.385) (end 131 36) (width 0.2) (layer F.Cu) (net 4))
 (segment (start 149 30.887501) (end 149 29.725) (width 0.2) (layer F.Cu) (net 4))
 (segment (start 148.725 35.1932) (end 148.725 31.162501) (width 0.2) (layer F.Cu) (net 4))
 (segment (start 148.0932 35.825) (end 148.725 35.1932) (width 0.2) (layer F.Cu) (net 4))
 (segment (start 133.675 35.825) (end 148.0932 35.825) (width 0.2) (layer F.Cu) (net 4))
 (segment (start 148.725 31.162501) (end 149 30.887501) (width 0.2) (layer F.Cu) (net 4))
 (segment (start 133.5 36) (end 133.675 35.825) (width 0.2) (layer F.Cu) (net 4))
 (segment (start 132.5 36) (end 133.5 36) (width 0.2) (layer F.Cu) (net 4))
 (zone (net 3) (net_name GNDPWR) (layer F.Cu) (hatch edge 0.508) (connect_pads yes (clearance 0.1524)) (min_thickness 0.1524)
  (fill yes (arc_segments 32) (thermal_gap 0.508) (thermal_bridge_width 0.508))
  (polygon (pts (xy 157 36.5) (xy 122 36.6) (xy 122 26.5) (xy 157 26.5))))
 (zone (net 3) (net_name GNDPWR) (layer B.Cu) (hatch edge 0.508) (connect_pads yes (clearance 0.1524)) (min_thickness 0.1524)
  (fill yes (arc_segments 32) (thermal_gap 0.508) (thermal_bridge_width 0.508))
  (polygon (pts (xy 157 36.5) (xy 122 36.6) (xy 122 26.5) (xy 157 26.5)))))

